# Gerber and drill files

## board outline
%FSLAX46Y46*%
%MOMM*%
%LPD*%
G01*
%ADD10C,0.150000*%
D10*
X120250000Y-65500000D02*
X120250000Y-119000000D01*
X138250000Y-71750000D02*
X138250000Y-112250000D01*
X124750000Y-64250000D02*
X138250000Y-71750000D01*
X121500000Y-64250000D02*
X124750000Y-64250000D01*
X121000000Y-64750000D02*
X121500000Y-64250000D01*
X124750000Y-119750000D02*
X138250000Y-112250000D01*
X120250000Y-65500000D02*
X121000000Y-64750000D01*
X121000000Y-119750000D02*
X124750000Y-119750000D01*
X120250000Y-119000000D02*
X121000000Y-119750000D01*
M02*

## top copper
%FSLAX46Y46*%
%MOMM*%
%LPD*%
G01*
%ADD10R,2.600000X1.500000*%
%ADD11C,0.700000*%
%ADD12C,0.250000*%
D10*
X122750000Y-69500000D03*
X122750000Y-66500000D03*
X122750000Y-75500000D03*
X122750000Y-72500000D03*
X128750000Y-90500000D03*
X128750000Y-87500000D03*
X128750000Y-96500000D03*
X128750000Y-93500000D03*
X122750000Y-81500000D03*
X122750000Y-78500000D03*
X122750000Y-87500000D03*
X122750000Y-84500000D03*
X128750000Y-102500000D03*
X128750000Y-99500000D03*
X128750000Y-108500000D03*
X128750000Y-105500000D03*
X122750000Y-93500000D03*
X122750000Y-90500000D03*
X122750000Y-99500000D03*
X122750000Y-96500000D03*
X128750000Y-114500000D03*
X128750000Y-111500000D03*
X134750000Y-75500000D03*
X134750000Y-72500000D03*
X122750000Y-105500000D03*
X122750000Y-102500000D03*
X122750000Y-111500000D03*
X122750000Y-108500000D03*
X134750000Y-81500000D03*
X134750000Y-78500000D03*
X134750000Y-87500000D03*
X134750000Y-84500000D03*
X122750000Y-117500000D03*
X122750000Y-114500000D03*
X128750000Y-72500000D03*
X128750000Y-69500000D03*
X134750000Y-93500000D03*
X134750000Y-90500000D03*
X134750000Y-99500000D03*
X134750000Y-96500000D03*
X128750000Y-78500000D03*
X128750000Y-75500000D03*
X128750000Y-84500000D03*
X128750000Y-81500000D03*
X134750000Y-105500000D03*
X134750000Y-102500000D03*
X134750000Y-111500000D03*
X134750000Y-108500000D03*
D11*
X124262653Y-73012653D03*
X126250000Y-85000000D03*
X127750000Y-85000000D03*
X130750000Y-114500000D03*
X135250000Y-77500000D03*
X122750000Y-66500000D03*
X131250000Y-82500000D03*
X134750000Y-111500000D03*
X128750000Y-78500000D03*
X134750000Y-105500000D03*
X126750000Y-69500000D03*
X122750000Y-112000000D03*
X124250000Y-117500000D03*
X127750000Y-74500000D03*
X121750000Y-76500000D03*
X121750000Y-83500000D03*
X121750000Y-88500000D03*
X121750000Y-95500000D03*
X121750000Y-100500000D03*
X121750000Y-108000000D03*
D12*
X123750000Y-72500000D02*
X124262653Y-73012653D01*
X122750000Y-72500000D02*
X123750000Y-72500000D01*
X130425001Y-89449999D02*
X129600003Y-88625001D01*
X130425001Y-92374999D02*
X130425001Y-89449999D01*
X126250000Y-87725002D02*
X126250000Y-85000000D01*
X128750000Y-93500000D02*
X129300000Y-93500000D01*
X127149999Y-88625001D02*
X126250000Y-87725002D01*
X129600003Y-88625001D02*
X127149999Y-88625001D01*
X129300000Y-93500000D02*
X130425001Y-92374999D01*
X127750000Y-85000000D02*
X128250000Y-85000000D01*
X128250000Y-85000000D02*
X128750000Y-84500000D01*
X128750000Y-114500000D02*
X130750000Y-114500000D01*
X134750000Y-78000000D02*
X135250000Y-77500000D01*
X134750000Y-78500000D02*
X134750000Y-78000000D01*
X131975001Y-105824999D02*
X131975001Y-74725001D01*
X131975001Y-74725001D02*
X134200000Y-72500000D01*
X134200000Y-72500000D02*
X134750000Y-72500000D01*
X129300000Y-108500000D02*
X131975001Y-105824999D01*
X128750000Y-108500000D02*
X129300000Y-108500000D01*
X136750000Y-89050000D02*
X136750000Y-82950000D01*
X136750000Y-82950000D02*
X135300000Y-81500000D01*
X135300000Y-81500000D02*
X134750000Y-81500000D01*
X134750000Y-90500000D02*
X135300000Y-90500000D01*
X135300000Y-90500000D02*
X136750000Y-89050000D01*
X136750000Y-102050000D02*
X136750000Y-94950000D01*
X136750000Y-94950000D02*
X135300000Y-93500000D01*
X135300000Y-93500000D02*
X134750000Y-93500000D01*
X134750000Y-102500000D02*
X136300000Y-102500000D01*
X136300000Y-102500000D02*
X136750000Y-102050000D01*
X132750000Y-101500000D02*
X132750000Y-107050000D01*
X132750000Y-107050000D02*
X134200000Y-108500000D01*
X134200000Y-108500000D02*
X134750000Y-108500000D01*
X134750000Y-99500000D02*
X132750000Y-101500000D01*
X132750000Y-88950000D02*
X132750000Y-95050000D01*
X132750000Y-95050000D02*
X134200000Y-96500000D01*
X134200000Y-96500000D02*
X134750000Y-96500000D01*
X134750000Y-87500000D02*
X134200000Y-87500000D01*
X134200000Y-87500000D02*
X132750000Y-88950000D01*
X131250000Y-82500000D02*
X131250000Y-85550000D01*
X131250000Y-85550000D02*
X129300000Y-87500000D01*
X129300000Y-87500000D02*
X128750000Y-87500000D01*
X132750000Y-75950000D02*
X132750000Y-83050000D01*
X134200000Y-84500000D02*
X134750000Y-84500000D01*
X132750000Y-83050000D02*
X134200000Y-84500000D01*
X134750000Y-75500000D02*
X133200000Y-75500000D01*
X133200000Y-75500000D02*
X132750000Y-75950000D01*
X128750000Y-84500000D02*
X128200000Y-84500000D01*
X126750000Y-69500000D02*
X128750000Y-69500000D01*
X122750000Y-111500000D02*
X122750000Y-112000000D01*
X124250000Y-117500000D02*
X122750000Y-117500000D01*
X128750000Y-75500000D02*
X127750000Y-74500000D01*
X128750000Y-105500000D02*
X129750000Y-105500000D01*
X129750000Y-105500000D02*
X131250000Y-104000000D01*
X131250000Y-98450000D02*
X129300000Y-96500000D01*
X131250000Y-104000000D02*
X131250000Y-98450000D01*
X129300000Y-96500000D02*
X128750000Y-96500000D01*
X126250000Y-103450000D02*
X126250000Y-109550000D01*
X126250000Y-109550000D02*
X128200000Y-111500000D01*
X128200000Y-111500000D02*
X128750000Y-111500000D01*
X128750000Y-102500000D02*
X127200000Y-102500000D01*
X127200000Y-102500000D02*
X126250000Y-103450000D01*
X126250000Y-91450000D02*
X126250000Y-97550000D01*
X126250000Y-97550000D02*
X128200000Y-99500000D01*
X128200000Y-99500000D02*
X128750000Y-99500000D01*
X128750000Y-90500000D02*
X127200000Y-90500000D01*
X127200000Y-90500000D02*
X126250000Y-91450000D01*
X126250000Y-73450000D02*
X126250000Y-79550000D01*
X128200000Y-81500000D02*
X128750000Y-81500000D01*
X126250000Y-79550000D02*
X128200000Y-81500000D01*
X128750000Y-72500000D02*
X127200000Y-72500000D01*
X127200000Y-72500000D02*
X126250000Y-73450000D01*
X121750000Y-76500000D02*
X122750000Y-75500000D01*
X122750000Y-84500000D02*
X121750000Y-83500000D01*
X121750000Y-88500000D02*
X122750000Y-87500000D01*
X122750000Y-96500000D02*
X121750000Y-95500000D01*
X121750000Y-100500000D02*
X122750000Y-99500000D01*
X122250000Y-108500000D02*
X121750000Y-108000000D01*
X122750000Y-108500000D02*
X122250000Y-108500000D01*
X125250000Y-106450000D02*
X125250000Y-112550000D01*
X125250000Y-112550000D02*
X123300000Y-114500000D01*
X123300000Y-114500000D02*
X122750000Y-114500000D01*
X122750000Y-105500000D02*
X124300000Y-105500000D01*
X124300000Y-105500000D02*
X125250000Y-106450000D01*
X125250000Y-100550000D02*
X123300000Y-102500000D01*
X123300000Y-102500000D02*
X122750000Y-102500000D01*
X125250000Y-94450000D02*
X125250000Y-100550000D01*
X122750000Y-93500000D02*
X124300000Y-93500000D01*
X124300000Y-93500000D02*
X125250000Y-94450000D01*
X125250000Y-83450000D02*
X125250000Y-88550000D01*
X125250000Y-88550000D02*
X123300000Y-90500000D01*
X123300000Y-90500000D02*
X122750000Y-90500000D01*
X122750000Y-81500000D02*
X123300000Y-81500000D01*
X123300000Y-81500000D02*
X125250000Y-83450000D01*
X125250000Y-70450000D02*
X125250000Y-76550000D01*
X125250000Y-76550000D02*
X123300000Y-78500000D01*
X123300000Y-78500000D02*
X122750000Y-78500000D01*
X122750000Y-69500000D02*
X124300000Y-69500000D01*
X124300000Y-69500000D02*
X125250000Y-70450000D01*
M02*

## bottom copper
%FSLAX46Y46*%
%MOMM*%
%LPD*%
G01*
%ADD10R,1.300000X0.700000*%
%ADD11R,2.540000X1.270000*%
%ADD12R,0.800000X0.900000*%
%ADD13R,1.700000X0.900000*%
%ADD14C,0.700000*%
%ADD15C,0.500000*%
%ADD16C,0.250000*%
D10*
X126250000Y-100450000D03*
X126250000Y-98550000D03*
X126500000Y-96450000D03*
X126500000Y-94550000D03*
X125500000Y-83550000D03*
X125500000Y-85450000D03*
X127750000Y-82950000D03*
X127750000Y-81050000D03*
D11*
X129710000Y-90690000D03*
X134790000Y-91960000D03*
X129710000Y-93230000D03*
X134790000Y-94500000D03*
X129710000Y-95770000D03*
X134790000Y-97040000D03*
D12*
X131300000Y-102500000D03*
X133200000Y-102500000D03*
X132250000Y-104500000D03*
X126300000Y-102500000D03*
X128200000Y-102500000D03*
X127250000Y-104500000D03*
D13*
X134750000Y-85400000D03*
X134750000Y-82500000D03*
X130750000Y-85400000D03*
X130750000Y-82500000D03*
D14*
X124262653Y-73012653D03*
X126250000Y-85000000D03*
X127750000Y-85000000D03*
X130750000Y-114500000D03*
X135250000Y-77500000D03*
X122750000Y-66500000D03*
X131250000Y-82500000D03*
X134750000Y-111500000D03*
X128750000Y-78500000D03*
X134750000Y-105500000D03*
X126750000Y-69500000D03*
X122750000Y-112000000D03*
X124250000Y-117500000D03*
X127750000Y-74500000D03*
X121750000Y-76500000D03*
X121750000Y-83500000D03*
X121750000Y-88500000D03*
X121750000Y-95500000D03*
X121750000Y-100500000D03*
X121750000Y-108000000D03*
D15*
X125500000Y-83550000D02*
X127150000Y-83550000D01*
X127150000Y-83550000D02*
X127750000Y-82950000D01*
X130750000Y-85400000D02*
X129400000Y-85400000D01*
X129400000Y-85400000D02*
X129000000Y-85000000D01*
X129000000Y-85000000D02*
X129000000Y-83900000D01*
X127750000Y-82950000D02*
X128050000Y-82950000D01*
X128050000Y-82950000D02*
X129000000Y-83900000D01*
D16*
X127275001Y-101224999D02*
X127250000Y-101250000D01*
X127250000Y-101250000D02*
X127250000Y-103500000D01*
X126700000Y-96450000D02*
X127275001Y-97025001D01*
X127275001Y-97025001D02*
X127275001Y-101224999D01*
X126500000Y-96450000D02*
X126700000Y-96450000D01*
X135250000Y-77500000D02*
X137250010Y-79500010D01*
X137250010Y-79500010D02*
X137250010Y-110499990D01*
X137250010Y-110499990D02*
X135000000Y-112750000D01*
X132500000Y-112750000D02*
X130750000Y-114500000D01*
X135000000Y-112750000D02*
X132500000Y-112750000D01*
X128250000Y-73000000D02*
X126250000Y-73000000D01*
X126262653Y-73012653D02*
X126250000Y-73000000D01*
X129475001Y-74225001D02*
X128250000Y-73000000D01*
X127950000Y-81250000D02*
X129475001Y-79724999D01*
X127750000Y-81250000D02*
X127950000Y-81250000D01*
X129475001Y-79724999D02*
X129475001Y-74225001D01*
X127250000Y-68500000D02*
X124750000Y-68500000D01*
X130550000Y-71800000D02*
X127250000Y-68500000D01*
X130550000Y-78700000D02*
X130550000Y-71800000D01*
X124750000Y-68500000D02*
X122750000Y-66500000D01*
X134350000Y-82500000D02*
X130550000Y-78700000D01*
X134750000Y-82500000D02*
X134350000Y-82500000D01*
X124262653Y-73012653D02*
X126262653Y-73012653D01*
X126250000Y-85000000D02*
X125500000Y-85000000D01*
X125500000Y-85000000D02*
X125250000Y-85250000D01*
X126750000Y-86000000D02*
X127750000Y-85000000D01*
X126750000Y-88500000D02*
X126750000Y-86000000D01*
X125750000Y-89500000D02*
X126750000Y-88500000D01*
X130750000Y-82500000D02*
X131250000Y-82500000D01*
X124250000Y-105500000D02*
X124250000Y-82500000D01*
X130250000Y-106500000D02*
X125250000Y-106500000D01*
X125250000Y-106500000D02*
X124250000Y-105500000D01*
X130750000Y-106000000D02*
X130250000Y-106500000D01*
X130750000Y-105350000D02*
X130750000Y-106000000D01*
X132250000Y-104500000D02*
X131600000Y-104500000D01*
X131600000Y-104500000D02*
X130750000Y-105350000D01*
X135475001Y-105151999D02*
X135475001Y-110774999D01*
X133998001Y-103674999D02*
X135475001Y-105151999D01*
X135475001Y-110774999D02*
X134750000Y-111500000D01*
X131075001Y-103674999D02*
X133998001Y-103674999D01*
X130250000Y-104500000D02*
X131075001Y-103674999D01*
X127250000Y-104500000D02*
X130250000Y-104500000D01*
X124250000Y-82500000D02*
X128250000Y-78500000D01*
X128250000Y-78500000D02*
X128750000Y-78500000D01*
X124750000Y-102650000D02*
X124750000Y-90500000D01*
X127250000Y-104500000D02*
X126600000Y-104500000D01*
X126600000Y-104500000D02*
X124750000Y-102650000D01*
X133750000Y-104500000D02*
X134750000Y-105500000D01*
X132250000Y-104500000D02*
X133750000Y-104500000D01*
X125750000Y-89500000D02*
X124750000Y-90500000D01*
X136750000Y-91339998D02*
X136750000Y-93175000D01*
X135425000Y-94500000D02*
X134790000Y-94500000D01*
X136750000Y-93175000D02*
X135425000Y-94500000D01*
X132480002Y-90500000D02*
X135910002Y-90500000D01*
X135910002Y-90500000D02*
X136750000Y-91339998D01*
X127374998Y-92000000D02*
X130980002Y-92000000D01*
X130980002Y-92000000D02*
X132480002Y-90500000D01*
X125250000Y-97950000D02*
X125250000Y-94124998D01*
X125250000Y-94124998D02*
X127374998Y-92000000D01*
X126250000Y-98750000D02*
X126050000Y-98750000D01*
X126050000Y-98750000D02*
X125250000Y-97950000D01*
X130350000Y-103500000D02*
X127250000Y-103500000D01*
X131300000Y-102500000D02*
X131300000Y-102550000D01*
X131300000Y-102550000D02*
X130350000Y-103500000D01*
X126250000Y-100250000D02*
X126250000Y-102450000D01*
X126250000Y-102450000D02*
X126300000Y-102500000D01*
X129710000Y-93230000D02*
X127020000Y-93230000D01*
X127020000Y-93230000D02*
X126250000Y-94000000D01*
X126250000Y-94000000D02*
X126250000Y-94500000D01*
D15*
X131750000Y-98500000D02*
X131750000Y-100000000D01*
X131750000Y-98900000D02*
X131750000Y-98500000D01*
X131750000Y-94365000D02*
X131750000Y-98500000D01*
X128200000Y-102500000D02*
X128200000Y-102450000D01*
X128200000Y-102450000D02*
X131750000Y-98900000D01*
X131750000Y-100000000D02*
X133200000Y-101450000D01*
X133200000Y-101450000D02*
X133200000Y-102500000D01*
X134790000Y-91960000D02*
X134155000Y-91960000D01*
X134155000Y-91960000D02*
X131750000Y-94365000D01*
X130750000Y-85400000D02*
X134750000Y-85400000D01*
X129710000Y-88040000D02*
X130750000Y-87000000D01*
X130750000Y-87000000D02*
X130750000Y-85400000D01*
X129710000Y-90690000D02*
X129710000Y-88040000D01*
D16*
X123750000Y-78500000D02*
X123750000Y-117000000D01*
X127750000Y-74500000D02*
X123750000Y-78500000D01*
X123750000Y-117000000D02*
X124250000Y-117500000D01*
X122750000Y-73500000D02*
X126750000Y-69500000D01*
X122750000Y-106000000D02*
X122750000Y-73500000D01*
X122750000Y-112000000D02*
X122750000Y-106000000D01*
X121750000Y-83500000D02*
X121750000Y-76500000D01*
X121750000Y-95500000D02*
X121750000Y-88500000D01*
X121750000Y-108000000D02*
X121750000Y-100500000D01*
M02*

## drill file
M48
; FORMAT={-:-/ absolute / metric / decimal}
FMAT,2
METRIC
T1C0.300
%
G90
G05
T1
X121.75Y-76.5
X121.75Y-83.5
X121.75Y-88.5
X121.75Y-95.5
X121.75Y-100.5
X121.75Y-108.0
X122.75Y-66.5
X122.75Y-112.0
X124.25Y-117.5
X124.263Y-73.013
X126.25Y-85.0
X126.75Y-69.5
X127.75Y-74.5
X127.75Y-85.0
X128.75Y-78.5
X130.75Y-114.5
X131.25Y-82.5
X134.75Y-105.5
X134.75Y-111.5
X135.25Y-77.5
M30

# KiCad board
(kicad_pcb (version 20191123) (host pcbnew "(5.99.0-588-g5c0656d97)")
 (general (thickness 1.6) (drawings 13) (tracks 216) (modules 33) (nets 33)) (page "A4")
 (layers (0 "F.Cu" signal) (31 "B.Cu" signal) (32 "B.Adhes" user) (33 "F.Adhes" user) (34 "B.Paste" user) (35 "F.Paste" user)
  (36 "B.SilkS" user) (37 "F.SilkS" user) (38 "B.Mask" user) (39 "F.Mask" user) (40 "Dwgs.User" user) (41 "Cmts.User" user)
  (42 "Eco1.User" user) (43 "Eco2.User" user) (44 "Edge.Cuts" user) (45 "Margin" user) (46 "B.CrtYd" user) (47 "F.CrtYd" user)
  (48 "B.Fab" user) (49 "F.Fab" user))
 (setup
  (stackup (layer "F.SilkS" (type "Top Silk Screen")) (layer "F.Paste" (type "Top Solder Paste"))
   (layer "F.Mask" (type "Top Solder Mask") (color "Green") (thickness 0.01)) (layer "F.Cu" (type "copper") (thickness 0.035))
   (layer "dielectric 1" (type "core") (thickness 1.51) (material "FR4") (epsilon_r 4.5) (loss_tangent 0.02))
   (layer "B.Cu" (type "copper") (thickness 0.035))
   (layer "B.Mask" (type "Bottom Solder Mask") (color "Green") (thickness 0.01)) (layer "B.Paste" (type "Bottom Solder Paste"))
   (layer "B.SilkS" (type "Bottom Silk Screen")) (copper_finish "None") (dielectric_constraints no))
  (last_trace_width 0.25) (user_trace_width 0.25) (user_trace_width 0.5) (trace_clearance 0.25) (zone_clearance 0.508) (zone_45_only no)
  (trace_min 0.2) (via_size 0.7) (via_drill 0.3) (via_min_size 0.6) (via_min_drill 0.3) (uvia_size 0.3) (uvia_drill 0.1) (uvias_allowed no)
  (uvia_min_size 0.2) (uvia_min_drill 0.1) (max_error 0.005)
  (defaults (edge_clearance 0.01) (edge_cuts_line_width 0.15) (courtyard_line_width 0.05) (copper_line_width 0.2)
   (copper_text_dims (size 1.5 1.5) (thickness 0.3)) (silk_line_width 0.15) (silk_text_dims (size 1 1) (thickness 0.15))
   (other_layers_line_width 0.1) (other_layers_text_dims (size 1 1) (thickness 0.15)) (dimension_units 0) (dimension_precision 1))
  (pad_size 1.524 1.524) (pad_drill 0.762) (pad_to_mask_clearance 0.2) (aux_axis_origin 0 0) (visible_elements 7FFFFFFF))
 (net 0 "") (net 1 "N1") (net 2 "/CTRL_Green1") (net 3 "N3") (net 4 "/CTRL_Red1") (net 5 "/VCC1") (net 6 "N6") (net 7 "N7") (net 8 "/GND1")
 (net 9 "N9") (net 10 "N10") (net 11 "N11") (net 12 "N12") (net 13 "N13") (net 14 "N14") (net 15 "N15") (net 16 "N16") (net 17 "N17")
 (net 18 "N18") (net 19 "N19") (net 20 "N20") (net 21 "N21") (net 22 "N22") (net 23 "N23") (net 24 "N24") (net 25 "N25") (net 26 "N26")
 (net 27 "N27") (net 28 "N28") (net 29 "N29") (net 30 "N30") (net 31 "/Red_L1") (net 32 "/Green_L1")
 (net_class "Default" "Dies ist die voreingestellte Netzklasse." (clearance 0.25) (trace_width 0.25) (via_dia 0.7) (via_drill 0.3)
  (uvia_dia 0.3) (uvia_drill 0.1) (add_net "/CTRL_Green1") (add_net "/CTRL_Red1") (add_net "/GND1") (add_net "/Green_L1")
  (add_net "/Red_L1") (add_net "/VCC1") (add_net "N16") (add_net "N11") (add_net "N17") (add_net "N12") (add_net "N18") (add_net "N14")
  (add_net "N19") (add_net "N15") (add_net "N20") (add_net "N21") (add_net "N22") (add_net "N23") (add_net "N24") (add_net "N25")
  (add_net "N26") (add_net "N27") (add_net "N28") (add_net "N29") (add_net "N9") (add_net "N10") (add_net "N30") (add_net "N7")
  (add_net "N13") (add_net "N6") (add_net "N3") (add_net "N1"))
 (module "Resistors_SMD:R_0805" (layer "B.Cu") (at 126.25 99.5 90)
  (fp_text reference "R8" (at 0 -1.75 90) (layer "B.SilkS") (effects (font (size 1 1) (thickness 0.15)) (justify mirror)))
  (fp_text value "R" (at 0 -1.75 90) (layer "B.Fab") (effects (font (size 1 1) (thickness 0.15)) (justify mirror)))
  (pad "1" smd rect (at -0.95 0 90) (size 0.7 1.3) (layers "B.Cu" "B.Paste" "B.Mask") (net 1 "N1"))
  (pad "2" smd rect (at 0.95 0 90) (size 0.7 1.3) (layers "B.Cu" "B.Paste" "B.Mask") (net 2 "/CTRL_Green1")))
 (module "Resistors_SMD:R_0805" (layer "B.Cu") (at 126.5 95.5 90)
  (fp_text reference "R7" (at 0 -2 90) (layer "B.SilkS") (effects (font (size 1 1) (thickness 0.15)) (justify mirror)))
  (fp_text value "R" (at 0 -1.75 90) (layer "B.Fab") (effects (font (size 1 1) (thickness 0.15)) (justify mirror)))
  (pad "1" smd rect (at -0.95 0 90) (size 0.7 1.3) (layers "B.Cu" "B.Paste" "B.Mask") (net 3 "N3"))
  (pad "2" smd rect (at 0.95 0 90) (size 0.7 1.3) (layers "B.Cu" "B.Paste" "B.Mask") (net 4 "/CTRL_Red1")))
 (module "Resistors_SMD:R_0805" (layer "B.Cu") (at 125.5 84.5 -90)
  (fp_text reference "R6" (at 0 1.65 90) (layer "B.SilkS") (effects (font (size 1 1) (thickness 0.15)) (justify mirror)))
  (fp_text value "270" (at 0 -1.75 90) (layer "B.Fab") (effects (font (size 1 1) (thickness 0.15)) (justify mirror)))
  (pad "1" smd rect (at -0.95 0 270) (size 0.7 1.3) (layers "B.Cu" "B.Paste" "B.Mask") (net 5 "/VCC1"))
  (pad "2" smd rect (at 0.95 0 270) (size 0.7 1.3) (layers "B.Cu" "B.Paste" "B.Mask") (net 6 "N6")))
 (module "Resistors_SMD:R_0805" (layer "B.Cu") (at 127.75 82 90)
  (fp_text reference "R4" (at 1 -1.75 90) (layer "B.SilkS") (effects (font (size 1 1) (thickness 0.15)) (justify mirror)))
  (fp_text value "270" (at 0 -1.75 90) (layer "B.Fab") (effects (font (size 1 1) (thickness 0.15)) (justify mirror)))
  (pad "1" smd rect (at -0.95 0 90) (size 0.7 1.3) (layers "B.Cu" "B.Paste" "B.Mask") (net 5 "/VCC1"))
  (pad "2" smd rect (at 0.95 0 90) (size 0.7 1.3) (layers "B.Cu" "B.Paste" "B.Mask") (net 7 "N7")))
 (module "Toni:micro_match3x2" (layer "B.Cu") (at 132.25 94.5 -90)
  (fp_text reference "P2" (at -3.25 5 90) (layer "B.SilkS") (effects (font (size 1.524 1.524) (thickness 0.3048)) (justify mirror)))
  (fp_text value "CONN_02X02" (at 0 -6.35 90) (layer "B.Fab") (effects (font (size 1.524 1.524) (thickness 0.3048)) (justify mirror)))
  (pad "1" smd rect (at -3.81 2.54 270) (size 1.27 2.54) (layers "B.Cu" "B.Paste" "B.Mask") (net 5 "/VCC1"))
  (pad "2" smd rect (at -2.54 -2.54 270) (size 1.27 2.54) (layers "B.Cu" "B.Paste" "B.Mask") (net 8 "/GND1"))
  (pad "3" smd rect (at -1.27 2.54 270) (size 1.27 2.54) (layers "B.Cu" "B.Paste" "B.Mask") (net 4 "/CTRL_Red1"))
  (pad "4" smd rect (at 0 -2.54 270) (size 1.27 2.54) (layers "B.Cu" "B.Paste" "B.Mask") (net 2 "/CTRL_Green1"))
  (pad "5" smd rect (at 1.27 2.54 270) (size 1.27 2.54) (layers "B.Cu" "B.Paste" "B.Mask"))
  (pad "6" smd rect (at 2.54 -2.54 270) (size 1.27 2.54) (layers "B.Cu" "B.Paste" "B.Mask")))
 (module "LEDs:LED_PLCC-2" (layer "F.Cu") (at 122.75 68 90)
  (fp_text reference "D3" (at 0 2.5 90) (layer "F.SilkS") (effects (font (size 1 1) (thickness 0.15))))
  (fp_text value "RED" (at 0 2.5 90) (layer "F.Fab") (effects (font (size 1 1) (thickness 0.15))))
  (pad "1" smd rect (at -1.5 0 90) (size 1.5 2.6) (layers "F.Cu" "F.Paste" "F.Mask") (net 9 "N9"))
  (pad "2" smd rect (at 1.5 0 90) (size 1.5 2.6) (layers "F.Cu" "F.Paste" "F.Mask") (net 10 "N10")))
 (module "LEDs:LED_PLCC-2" (layer "F.Cu") (at 122.75 74 90)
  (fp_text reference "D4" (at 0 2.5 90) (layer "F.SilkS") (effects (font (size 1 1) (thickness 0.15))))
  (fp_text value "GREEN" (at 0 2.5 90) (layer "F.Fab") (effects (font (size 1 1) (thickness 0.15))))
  (pad "1" smd rect (at -1.5 0 90) (size 1.5 2.6) (layers "F.Cu" "F.Paste" "F.Mask") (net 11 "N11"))
  (pad "2" smd rect (at 1.5 0 90) (size 1.5 2.6) (layers "F.Cu" "F.Paste" "F.Mask") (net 7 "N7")))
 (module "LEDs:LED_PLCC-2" (layer "F.Cu") (at 128.75 89 90)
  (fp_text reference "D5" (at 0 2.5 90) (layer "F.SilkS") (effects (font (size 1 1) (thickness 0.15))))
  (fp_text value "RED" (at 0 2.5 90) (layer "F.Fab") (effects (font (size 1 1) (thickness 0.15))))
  (pad "1" smd rect (at -1.5 0 90) (size 1.5 2.6) (layers "F.Cu" "F.Paste" "F.Mask") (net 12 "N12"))
  (pad "2" smd rect (at 1.5 0 90) (size 1.5 2.6) (layers "F.Cu" "F.Paste" "F.Mask") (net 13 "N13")))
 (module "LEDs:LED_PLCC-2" (layer "F.Cu") (at 128.75 95 90)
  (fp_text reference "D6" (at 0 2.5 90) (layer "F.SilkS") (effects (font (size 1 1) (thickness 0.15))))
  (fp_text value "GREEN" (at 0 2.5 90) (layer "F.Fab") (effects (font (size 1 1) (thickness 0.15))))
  (pad "1" smd rect (at -1.5 0 90) (size 1.5 2.6) (layers "F.Cu" "F.Paste" "F.Mask") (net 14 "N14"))
  (pad "2" smd rect (at 1.5 0 90) (size 1.5 2.6) (layers "F.Cu" "F.Paste" "F.Mask") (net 6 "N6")))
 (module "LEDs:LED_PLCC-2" (layer "F.Cu") (at 122.75 80 90)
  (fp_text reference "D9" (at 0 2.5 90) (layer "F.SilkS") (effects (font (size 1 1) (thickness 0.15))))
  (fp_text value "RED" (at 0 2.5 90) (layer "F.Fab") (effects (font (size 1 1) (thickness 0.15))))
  (pad "1" smd rect (at -1.5 0 90) (size 1.5 2.6) (layers "F.Cu" "F.Paste" "F.Mask") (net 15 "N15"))
  (pad "2" smd rect (at 1.5 0 90) (size 1.5 2.6) (layers "F.Cu" "F.Paste" "F.Mask") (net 9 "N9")))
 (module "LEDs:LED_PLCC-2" (layer "F.Cu") (at 122.75 86 90)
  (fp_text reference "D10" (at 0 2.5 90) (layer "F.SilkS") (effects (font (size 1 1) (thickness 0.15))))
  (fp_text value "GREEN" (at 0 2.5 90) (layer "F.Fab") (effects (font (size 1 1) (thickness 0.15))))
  (pad "1" smd rect (at -1.5 0 90) (size 1.5 2.6) (layers "F.Cu" "F.Paste" "F.Mask") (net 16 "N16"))
  (pad "2" smd rect (at 1.5 0 90) (size 1.5 2.6) (layers "F.Cu" "F.Paste" "F.Mask") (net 11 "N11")))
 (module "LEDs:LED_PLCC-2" (layer "F.Cu") (at 128.75 101 90)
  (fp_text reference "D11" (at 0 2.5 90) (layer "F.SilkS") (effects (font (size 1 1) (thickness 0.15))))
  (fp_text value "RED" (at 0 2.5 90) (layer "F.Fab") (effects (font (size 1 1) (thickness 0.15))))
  (pad "1" smd rect (at -1.5 0 90) (size 1.5 2.6) (layers "F.Cu" "F.Paste" "F.Mask") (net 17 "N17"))
  (pad "2" smd rect (at 1.5 0 90) (size 1.5 2.6) (layers "F.Cu" "F.Paste" "F.Mask") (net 12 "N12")))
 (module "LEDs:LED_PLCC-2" (layer "F.Cu") (at 128.75 107 90)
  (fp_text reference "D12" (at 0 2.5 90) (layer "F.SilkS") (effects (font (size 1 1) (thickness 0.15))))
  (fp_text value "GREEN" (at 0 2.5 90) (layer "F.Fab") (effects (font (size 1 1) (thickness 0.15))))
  (pad "1" smd rect (at -1.5 0 90) (size 1.5 2.6) (layers "F.Cu" "F.Paste" "F.Mask") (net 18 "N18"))
  (pad "2" smd rect (at 1.5 0 90) (size 1.5 2.6) (layers "F.Cu" "F.Paste" "F.Mask") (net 14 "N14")))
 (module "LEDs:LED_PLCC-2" (layer "F.Cu") (at 122.75 92 90)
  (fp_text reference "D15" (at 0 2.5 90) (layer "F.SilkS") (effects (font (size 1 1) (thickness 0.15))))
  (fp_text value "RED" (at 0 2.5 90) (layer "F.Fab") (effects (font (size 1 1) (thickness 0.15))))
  (pad "1" smd rect (at -1.5 0 90) (size 1.5 2.6) (layers "F.Cu" "F.Paste" "F.Mask") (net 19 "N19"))
  (pad "2" smd rect (at 1.5 0 90) (size 1.5 2.6) (layers "F.Cu" "F.Paste" "F.Mask") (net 15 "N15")))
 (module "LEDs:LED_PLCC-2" (layer "F.Cu") (at 122.75 98 90)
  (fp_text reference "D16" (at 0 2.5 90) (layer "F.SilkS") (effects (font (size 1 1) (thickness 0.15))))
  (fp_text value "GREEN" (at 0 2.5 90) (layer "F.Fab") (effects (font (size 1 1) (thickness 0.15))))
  (pad "1" smd rect (at -1.5 0 90) (size 1.5 2.6) (layers "F.Cu" "F.Paste" "F.Mask") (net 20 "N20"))
  (pad "2" smd rect (at 1.5 0 90) (size 1.5 2.6) (layers "F.Cu" "F.Paste" "F.Mask") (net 16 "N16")))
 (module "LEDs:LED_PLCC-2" (layer "F.Cu") (at 128.75 113 90)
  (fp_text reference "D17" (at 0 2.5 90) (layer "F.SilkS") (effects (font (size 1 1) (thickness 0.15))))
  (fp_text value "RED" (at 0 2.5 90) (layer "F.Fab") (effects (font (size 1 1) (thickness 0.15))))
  (pad "1" smd rect (at -1.5 0 90) (size 1.5 2.6) (layers "F.Cu" "F.Paste" "F.Mask") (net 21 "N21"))
  (pad "2" smd rect (at 1.5 0 90) (size 1.5 2.6) (layers "F.Cu" "F.Paste" "F.Mask") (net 17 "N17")))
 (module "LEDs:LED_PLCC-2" (layer "F.Cu") (at 134.75 74 90)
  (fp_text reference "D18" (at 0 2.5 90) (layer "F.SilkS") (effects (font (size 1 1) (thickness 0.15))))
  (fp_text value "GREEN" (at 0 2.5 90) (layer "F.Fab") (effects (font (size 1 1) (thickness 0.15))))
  (pad "1" smd rect (at -1.5 0 90) (size 1.5 2.6) (layers "F.Cu" "F.Paste" "F.Mask") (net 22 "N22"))
  (pad "2" smd rect (at 1.5 0 90) (size 1.5 2.6) (layers "F.Cu" "F.Paste" "F.Mask") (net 18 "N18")))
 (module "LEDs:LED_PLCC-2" (layer "F.Cu") (at 122.75 104 90)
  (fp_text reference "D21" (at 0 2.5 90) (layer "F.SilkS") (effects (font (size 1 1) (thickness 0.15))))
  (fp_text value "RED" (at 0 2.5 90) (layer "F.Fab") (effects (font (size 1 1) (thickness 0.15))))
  (pad "1" smd rect (at -1.5 0 90) (size 1.5 2.6) (layers "F.Cu" "F.Paste" "F.Mask") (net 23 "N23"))
  (pad "2" smd rect (at 1.5 0 90) (size 1.5 2.6) (layers "F.Cu" "F.Paste" "F.Mask") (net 19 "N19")))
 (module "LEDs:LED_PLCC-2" (layer "F.Cu") (at 122.75 110 90)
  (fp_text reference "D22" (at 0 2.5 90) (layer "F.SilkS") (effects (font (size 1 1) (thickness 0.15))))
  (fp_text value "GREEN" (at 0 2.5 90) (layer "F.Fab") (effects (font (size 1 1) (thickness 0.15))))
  (pad "1" smd rect (at -1.5 0 90) (size 1.5 2.6) (layers "F.Cu" "F.Paste" "F.Mask") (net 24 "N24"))
  (pad "2" smd rect (at 1.5 0 90) (size 1.5 2.6) (layers "F.Cu" "F.Paste" "F.Mask") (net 20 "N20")))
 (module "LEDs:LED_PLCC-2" (layer "F.Cu") (at 134.75 80 90)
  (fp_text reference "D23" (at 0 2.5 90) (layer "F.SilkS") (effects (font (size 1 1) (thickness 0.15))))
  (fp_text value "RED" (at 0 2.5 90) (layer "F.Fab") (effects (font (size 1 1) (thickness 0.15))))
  (pad "1" smd rect (at -1.5 0 90) (size 1.5 2.6) (layers "F.Cu" "F.Paste" "F.Mask") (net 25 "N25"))
  (pad "2" smd rect (at 1.5 0 90) (size 1.5 2.6) (layers "F.Cu" "F.Paste" "F.Mask") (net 21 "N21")))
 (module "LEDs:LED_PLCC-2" (layer "F.Cu") (at 134.75 86 90)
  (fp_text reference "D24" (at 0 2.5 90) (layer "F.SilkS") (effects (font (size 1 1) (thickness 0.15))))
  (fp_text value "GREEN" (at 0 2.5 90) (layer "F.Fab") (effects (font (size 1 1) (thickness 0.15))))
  (pad "1" smd rect (at -1.5 0 90) (size 1.5 2.6) (layers "F.Cu" "F.Paste" "F.Mask") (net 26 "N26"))
  (pad "2" smd rect (at 1.5 0 90) (size 1.5 2.6) (layers "F.Cu" "F.Paste" "F.Mask") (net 22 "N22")))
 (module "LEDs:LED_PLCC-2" (layer "F.Cu") (at 122.75 116 90)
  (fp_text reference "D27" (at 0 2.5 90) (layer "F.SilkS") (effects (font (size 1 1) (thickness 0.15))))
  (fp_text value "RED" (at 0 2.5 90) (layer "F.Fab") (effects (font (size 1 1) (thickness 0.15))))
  (pad "1" smd rect (at -1.5 0 90) (size 1.5 2.6) (layers "F.Cu" "F.Paste" "F.Mask") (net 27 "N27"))
  (pad "2" smd rect (at 1.5 0 90) (size 1.5 2.6) (layers "F.Cu" "F.Paste" "F.Mask") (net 23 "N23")))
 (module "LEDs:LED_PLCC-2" (layer "F.Cu") (at 128.75 71 90)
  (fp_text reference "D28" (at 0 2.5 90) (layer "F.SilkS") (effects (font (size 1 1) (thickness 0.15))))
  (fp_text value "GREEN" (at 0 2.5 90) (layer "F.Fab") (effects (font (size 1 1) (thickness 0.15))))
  (pad "1" smd rect (at -1.5 0 90) (size 1.5 2.6) (layers "F.Cu" "F.Paste" "F.Mask") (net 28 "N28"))
  (pad "2" smd rect (at 1.5 0 90) (size 1.5 2.6) (layers "F.Cu" "F.Paste" "F.Mask") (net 24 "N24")))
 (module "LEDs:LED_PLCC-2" (layer "F.Cu") (at 134.75 92 90)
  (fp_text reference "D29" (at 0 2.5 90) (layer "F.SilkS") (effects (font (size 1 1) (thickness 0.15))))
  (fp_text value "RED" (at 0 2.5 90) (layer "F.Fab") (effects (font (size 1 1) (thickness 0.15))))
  (pad "1" smd rect (at -1.5 0 90) (size 1.5 2.6) (layers "F.Cu" "F.Paste" "F.Mask") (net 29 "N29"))
  (pad "2" smd rect (at 1.5 0 90) (size 1.5 2.6) (layers "F.Cu" "F.Paste" "F.Mask") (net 25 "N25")))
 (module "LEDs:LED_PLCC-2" (layer "F.Cu") (at 134.75 98 90)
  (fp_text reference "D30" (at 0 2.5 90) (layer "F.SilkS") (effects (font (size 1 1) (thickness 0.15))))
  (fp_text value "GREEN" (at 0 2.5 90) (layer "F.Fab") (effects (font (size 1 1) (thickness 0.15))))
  (pad "1" smd rect (at -1.5 0 90) (size 1.5 2.6) (layers "F.Cu" "F.Paste" "F.Mask") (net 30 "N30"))
  (pad "2" smd rect (at 1.5 0 90) (size 1.5 2.6) (layers "F.Cu" "F.Paste" "F.Mask") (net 26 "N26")))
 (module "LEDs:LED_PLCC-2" (layer "F.Cu") (at 128.75 77 90)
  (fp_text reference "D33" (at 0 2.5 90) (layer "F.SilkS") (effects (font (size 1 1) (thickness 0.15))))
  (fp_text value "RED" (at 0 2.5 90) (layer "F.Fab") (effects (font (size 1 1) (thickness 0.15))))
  (pad "1" smd rect (at -1.5 0 90) (size 1.5 2.6) (layers "F.Cu" "F.Paste" "F.Mask") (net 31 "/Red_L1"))
  (pad "2" smd rect (at 1.5 0 90) (size 1.5 2.6) (layers "F.Cu" "F.Paste" "F.Mask") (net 27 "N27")))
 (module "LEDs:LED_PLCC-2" (layer "F.Cu") (at 128.75 83 90)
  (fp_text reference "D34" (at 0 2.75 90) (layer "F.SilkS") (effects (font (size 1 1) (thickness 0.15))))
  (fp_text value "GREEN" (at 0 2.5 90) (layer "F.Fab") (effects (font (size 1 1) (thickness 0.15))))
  (pad "1" smd rect (at -1.5 0 90) (size 1.5 2.6) (layers "F.Cu" "F.Paste" "F.Mask") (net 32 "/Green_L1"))
  (pad "2" smd rect (at 1.5 0 90) (size 1.5 2.6) (layers "F.Cu" "F.Paste" "F.Mask") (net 28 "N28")))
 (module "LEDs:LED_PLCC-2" (layer "F.Cu") (at 134.75 104 90)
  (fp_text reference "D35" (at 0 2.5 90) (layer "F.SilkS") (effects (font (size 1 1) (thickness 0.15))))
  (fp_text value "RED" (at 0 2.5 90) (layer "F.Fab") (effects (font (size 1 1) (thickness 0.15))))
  (pad "1" smd rect (at -1.5 0 90) (size 1.5 2.6) (layers "F.Cu" "F.Paste" "F.Mask") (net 31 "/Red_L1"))
  (pad "2" smd rect (at 1.5 0 90) (size 1.5 2.6) (layers "F.Cu" "F.Paste" "F.Mask") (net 29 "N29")))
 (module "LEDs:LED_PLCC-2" (layer "F.Cu") (at 134.75 110 90)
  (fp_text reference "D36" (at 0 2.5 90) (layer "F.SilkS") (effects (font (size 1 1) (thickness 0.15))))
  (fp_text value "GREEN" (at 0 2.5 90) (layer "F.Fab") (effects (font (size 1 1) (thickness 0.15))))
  (pad "1" smd rect (at -1.5 0 90) (size 1.5 2.6) (layers "F.Cu" "F.Paste" "F.Mask") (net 32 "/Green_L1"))
  (pad "2" smd rect (at 1.5 0 90) (size 1.5 2.6) (layers "F.Cu" "F.Paste" "F.Mask") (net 30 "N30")))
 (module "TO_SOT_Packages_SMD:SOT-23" (layer "B.Cu") (at 132.25 103.5 -90)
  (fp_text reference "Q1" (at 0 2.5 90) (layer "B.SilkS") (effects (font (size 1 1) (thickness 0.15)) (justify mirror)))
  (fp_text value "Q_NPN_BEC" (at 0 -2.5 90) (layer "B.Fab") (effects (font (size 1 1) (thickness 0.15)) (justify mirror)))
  (pad "1" smd rect (at -1 0.95 270) (size 0.9 0.8) (layers "B.Cu" "B.Paste" "B.Mask") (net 3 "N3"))
  (pad "2" smd rect (at -1 -0.95 270) (size 0.9 0.8) (layers "B.Cu" "B.Paste" "B.Mask") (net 8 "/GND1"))
  (pad "3" smd rect (at 1 0 270) (size 0.9 0.8) (layers "B.Cu" "B.Paste" "B.Mask") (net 31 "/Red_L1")))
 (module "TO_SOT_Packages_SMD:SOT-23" (layer "B.Cu") (at 127.25 103.5 -90)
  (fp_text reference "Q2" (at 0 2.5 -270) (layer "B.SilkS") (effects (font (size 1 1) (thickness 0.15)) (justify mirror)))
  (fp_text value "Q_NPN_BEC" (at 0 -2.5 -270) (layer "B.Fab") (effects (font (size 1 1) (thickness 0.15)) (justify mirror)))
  (pad "1" smd rect (at -1 0.95 270) (size 0.9 0.8) (layers "B.Cu" "B.Paste" "B.Mask") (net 1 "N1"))
  (pad "2" smd rect (at -1 -0.95 270) (size 0.9 0.8) (layers "B.Cu" "B.Paste" "B.Mask") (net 8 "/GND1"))
  (pad "3" smd rect (at 1 0 270) (size 0.9 0.8) (layers "B.Cu" "B.Paste" "B.Mask") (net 32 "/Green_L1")))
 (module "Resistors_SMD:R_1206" (layer "B.Cu") (at 134.75 83.95 90)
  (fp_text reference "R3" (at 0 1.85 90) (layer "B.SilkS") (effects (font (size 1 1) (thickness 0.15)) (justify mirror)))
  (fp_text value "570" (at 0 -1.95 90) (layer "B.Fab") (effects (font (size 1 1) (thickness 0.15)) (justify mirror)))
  (pad "1" smd rect (at -1.45 0 90) (size 0.9 1.7) (layers "B.Cu" "B.Paste" "B.Mask") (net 5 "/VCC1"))
  (pad "2" smd rect (at 1.45 0 90) (size 0.9 1.7) (layers "B.Cu" "B.Paste" "B.Mask") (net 10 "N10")))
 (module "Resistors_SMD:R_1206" (layer "B.Cu") (at 130.75 83.95 90)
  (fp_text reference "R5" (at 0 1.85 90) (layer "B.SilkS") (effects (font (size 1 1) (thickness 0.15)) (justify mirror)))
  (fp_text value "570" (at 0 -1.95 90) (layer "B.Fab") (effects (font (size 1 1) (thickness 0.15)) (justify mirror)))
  (pad "1" smd rect (at -1.45 0 90) (size 0.9 1.7) (layers "B.Cu" "B.Paste" "B.Mask") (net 5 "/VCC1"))
  (pad "2" smd rect (at 1.45 0 90) (size 0.9 1.7) (layers "B.Cu" "B.Paste" "B.Mask") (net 13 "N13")))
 (gr_line (start 120.25 65.5) (end 120.25 119) (layer "Edge.Cuts") (width 0.15))
 (gr_line (start 138.25 71.75) (end 138.25 112.25) (layer "Edge.Cuts") (width 0.15))
 (gr_line (start 124.75 64.25) (end 138.25 71.75) (layer "Edge.Cuts") (width 0.15))
 (gr_line (start 121.5 64.25) (end 124.75 64.25) (layer "Edge.Cuts") (width 0.15))
 (gr_line (start 121 64.75) (end 121.5 64.25) (layer "Edge.Cuts") (width 0.15))
 (gr_line (start 124.75 119.75) (end 138.25 112.25) (layer "Edge.Cuts") (width 0.15))
 (gr_line (start 120.25 65.5) (end 121 64.75) (layer "Edge.Cuts") (width 0.15))
 (gr_line (start 121 119.75) (end 124.75 119.75) (layer "Edge.Cuts") (width 0.15))
 (gr_line (start 120.25 119) (end 121 119.75) (layer "Edge.Cuts") (width 0.15))
 (segment (start 125.5 83.55) (end 127.15 83.55) (width 0.5) (layer "B.Cu") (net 5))
 (segment (start 127.15 83.55) (end 127.75 82.95) (width 0.5) (layer "B.Cu") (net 5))
 (segment (start 130.75 85.4) (end 129.4 85.4) (width 0.5) (layer "B.Cu") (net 5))
 (segment (start 129.4 85.4) (end 129 85) (width 0.5) (layer "B.Cu") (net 5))
 (segment (start 129 85) (end 129 83.9) (width 0.5) (layer "B.Cu") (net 5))
 (segment (start 127.75 82.95) (end 128.05 82.95) (width 0.5) (layer "B.Cu") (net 5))
 (segment (start 128.05 82.95) (end 129 83.9) (width 0.5) (layer "B.Cu") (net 5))
 (segment (start 127.275001 101.224999) (end 127.25 101.25) (width 0.25) (layer "B.Cu") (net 3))
 (segment (start 127.25 101.25) (end 127.25 103.5) (width 0.25) (layer "B.Cu") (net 3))
 (segment (start 126.7 96.45) (end 127.275001 97.025001) (width 0.25) (layer "B.Cu") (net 3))
 (segment (start 127.275001 97.025001) (end 127.275001 101.224999) (width 0.25) (layer "B.Cu") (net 3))
 (segment (start 126.5 96.45) (end 126.7 96.45) (width 0.25) (layer "B.Cu") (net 3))
 (segment (start 135.25 77.5) (end 137.25001 79.50001) (width 0.25) (layer "B.Cu") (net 21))
 (segment (start 137.25001 79.50001) (end 137.25001 110.49999) (width 0.25) (layer "B.Cu") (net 21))
 (segment (start 137.25001 110.49999) (end 135 112.75) (width 0.25) (layer "B.Cu") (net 21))
 (segment (start 132.5 112.75) (end 130.75 114.5) (width 0.25) (layer "B.Cu") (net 21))
 (segment (start 135 112.75) (end 132.5 112.75) (width 0.25) (layer "B.Cu") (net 21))
 (segment (start 128.25 73) (end 126.25 73) (width 0.25) (layer "B.Cu") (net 7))
 (segment (start 126.262653 73.012653) (end 126.25 73) (width 0.25) (layer "B.Cu") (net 7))
 (segment (start 129.475001 74.225001) (end 128.25 73) (width 0.25) (layer "B.Cu") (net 7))
 (segment (start 127.95 81.25) (end 129.475001 79.724999) (width 0.25) (layer "B.Cu") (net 7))
 (segment (start 127.75 81.25) (end 127.95 81.25) (width 0.25) (layer "B.Cu") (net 7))
 (segment (start 129.475001 79.724999) (end 129.475001 74.225001) (width 0.25) (layer "B.Cu") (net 7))
 (segment (start 127.25 68.5) (end 124.75 68.5) (width 0.25) (layer "B.Cu") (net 10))
 (segment (start 130.55 71.8) (end 127.25 68.5) (width 0.25) (layer "B.Cu") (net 10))
 (segment (start 130.55 78.7) (end 130.55 71.8) (width 0.25) (layer "B.Cu") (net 10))
 (segment (start 124.75 68.5) (end 122.75 66.5) (width 0.25) (layer "B.Cu") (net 10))
 (segment (start 134.35 82.5) (end 130.55 78.7) (width 0.25) (layer "B.Cu") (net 10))
 (segment (start 134.75 82.5) (end 134.35 82.5) (width 0.25) (layer "B.Cu") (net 10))
 (segment (start 124.262653 73.012653) (end 126.262653 73.012653) (width 0.25) (layer "B.Cu") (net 7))
 (segment (start 123.75 72.5) (end 124.262653 73.012653) (width 0.25) (layer "F.Cu") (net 7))
 (segment (start 122.75 72.5) (end 123.75 72.5) (width 0.25) (layer "F.Cu") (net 7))
 (via (at 124.262653 73.012653) (size 0.7) (drill 0.3) (layers "F.Cu" "B.Cu") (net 7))
 (segment (start 126.25 85) (end 125.5 85) (width 0.25) (layer "B.Cu") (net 6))
 (segment (start 125.5 85) (end 125.25 85.25) (width 0.25) (layer "B.Cu") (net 6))
 (segment (start 130.425001 89.449999) (end 129.600003 88.625001) (width 0.25) (layer "F.Cu") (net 6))
 (segment (start 130.425001 92.374999) (end 130.425001 89.449999) (width 0.25) (layer "F.Cu") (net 6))
 (segment (start 126.25 87.725002) (end 126.25 85) (width 0.25) (layer "F.Cu") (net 6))
 (via (at 126.25 85) (size 0.7) (drill 0.3) (layers "F.Cu" "B.Cu") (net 6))
 (segment (start 128.75 93.5) (end 129.3 93.5) (width 0.25) (layer "F.Cu") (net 6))
 (segment (start 127.149999 88.625001) (end 126.25 87.725002) (width 0.25) (layer "F.Cu") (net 6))
 (segment (start 129.600003 88.625001) (end 127.149999 88.625001) (width 0.25) (layer "F.Cu") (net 6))
 (segment (start 129.3 93.5) (end 130.425001 92.374999) (width 0.25) (layer "F.Cu") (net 6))
 (segment (start 127.75 85) (end 128.25 85) (width 0.25) (layer "F.Cu") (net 32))
 (segment (start 128.25 85) (end 128.75 84.5) (width 0.25) (layer "F.Cu") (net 32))
 (segment (start 126.75 86) (end 127.75 85) (width 0.25) (layer "B.Cu") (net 32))
 (via (at 127.75 85) (size 0.7) (drill 0.3) (layers "F.Cu" "B.Cu") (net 32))
 (segment (start 126.75 88.5) (end 126.75 86) (width 0.25) (layer "B.Cu") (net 32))
 (segment (start 125.75 89.5) (end 126.75 88.5) (width 0.25) (layer "B.Cu") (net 32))
 (segment (start 128.75 114.5) (end 130.75 114.5) (width 0.25) (layer "F.Cu") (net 21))
 (via (at 130.75 114.5) (size 0.7) (drill 0.3) (layers "F.Cu" "B.Cu") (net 21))
 (segment (start 134.75 78) (end 135.25 77.5) (width 0.25) (layer "F.Cu") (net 21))
 (via (at 135.25 77.5) (size 0.7) (drill 0.3) (layers "F.Cu" "B.Cu") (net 21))
 (segment (start 134.75 78.5) (end 134.75 78) (width 0.25) (layer "F.Cu") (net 21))
 (segment (start 131.975001 105.824999) (end 131.975001 74.725001) (width 0.25) (layer "F.Cu") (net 18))
 (segment (start 131.975001 74.725001) (end 134.2 72.5) (width 0.25) (layer "F.Cu") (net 18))
 (segment (start 134.2 72.5) (end 134.75 72.5) (width 0.25) (layer "F.Cu") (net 18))
 (segment (start 129.3 108.5) (end 131.975001 105.824999) (width 0.25) (layer "F.Cu") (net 18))
 (segment (start 128.75 108.5) (end 129.3 108.5) (width 0.25) (layer "F.Cu") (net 18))
 (segment (start 136.75 89.05) (end 136.75 82.95) (width 0.25) (layer "F.Cu") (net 25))
 (segment (start 136.75 82.95) (end 135.3 81.5) (width 0.25) (layer "F.Cu") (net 25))
 (segment (start 135.3 81.5) (end 134.75 81.5) (width 0.25) (layer "F.Cu") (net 25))
 (segment (start 134.75 90.5) (end 135.3 90.5) (width 0.25) (layer "F.Cu") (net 25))
 (segment (start 135.3 90.5) (end 136.75 89.05) (width 0.25) (layer "F.Cu") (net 25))
 (segment (start 136.75 102.05) (end 136.75 94.95) (width 0.25) (layer "F.Cu") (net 29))
 (segment (start 136.75 94.95) (end 135.3 93.5) (width 0.25) (layer "F.Cu") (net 29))
 (segment (start 135.3 93.5) (end 134.75 93.5) (width 0.25) (layer "F.Cu") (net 29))
 (segment (start 134.75 102.5) (end 136.3 102.5) (width 0.25) (layer "F.Cu") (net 29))
 (segment (start 136.3 102.5) (end 136.75 102.05) (width 0.25) (layer "F.Cu") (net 29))
 (segment (start 132.75 101.5) (end 132.75 107.05) (width 0.25) (layer "F.Cu") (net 30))
 (segment (start 132.75 107.05) (end 134.2 108.5) (width 0.25) (layer "F.Cu") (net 30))
 (segment (start 134.2 108.5) (end 134.75 108.5) (width 0.25) (layer "F.Cu") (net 30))
 (segment (start 134.75 99.5) (end 132.75 101.5) (width 0.25) (layer "F.Cu") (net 30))
 (segment (start 132.75 88.95) (end 132.75 95.05) (width 0.25) (layer "F.Cu") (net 26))
 (segment (start 132.75 95.05) (end 134.2 96.5) (width 0.25) (layer "F.Cu") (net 26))
 (segment (start 134.2 96.5) (end 134.75 96.5) (width 0.25) (layer "F.Cu") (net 26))
 (segment (start 134.75 87.5) (end 134.2 87.5) (width 0.25) (layer "F.Cu") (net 26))
 (segment (start 134.2 87.5) (end 132.75 88.95) (width 0.25) (layer "F.Cu") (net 26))
 (via (at 122.75 66.5) (size 0.7) (drill 0.3) (layers "F.Cu" "B.Cu") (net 10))
 (segment (start 131.25 82.5) (end 131.25 85.55) (width 0.25) (layer "F.Cu") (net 13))
 (segment (start 131.25 85.55) (end 129.3 87.5) (width 0.25) (layer "F.Cu") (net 13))
 (segment (start 129.3 87.5) (end 128.75 87.5) (width 0.25) (layer "F.Cu") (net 13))
 (segment (start 130.75 82.5) (end 131.25 82.5) (width 0.25) (layer "B.Cu") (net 13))
 (via (at 131.25 82.5) (size 0.7) (drill 0.3) (layers "F.Cu" "B.Cu") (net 13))
 (segment (start 132.75 75.95) (end 132.75 83.05) (width 0.25) (layer "F.Cu") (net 22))
 (segment (start 134.2 84.5) (end 134.75 84.5) (width 0.25) (layer "F.Cu") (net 22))
 (segment (start 132.75 83.05) (end 134.2 84.5) (width 0.25) (layer "F.Cu") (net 22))
 (segment (start 134.75 75.5) (end 133.2 75.5) (width 0.25) (layer "F.Cu") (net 22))
 (segment (start 133.2 75.5) (end 132.75 75.95) (width 0.25) (layer "F.Cu") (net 22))
 (segment (start 124.25 105.5) (end 124.25 82.5) (width 0.25) (layer "B.Cu") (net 31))
 (segment (start 130.25 106.5) (end 125.25 106.5) (width 0.25) (layer "B.Cu") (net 31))
 (segment (start 125.25 106.5) (end 124.25 105.5) (width 0.25) (layer "B.Cu") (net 31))
 (segment (start 130.75 106) (end 130.25 106.5) (width 0.25) (layer "B.Cu") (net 31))
 (segment (start 130.75 105.35) (end 130.75 106) (width 0.25) (layer "B.Cu") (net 31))
 (segment (start 132.25 104.5) (end 131.6 104.5) (width 0.25) (layer "B.Cu") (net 31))
 (segment (start 131.6 104.5) (end 130.75 105.35) (width 0.25) (layer "B.Cu") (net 31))
 (segment (start 135.475001 105.151999) (end 135.475001 110.774999) (width 0.25) (layer "B.Cu") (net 32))
 (segment (start 133.998001 103.674999) (end 135.475001 105.151999) (width 0.25) (layer "B.Cu") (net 32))
 (segment (start 135.475001 110.774999) (end 134.75 111.5) (width 0.25) (layer "B.Cu") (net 32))
 (segment (start 131.075001 103.674999) (end 133.998001 103.674999) (width 0.25) (layer "B.Cu") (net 32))
 (segment (start 130.25 104.5) (end 131.075001 103.674999) (width 0.25) (layer "B.Cu") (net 32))
 (via (at 134.75 111.5) (size 0.7) (drill 0.3) (layers "F.Cu" "B.Cu") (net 32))
 (segment (start 127.25 104.5) (end 130.25 104.5) (width 0.25) (layer "B.Cu") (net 32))
 (segment (start 124.25 82.5) (end 128.25 78.5) (width 0.25) (layer "B.Cu") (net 31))
 (segment (start 128.25 78.5) (end 128.75 78.5) (width 0.25) (layer "B.Cu") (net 31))
 (segment (start 124.75 102.65) (end 124.75 90.5) (width 0.25) (layer "B.Cu") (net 32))
 (segment (start 127.25 104.5) (end 126.6 104.5) (width 0.25) (layer "B.Cu") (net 32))
 (segment (start 126.6 104.5) (end 124.75 102.65) (width 0.25) (layer "B.Cu") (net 32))
 (via (at 128.75 78.5) (size 0.7) (drill 0.3) (layers "F.Cu" "B.Cu") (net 31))
 (segment (start 133.75 104.5) (end 134.75 105.5) (width 0.25) (layer "B.Cu") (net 31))
 (segment (start 132.25 104.5) (end 133.75 104.5) (width 0.25) (layer "B.Cu") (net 31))
 (via (at 134.75 105.5) (size 0.7) (drill 0.3) (layers "F.Cu" "B.Cu") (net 31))
 (segment (start 125.75 89.5) (end 124.75 90.5) (width 0.25) (layer "B.Cu") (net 32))
 (segment (start 128.75 84.5) (end 128.2 84.5) (width 0.25) (layer "F.Cu") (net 32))
 (segment (start 136.75 91.339998) (end 136.75 93.175) (width 0.25) (layer "B.Cu") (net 2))
 (segment (start 135.425 94.5) (end 134.79 94.5) (width 0.25) (layer "B.Cu") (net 2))
 (segment (start 136.75 93.175) (end 135.425 94.5) (width 0.25) (layer "B.Cu") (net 2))
 (segment (start 132.480002 90.5) (end 135.910002 90.5) (width 0.25) (layer "B.Cu") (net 2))
 (segment (start 135.910002 90.5) (end 136.75 91.339998) (width 0.25) (layer "B.Cu") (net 2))
 (segment (start 127.374998 92) (end 130.980002 92) (width 0.25) (layer "B.Cu") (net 2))
 (segment (start 130.980002 92) (end 132.480002 90.5) (width 0.25) (layer "B.Cu") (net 2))
 (segment (start 125.25 97.95) (end 125.25 94.124998) (width 0.25) (layer "B.Cu") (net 2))
 (segment (start 125.25 94.124998) (end 127.374998 92) (width 0.25) (layer "B.Cu") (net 2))
 (segment (start 126.25 98.75) (end 126.05 98.75) (width 0.25) (layer "B.Cu") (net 2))
 (segment (start 126.05 98.75) (end 125.25 97.95) (width 0.25) (layer "B.Cu") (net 2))
 (segment (start 130.35 103.5) (end 127.25 103.5) (width 0.25) (layer "B.Cu") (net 3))
 (segment (start 131.3 102.5) (end 131.3 102.55) (width 0.25) (layer "B.Cu") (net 3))
 (segment (start 131.3 102.55) (end 130.35 103.5) (width 0.25) (layer "B.Cu") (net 3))
 (segment (start 126.25 100.25) (end 126.25 102.45) (width 0.25) (layer "B.Cu") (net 1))
 (segment (start 126.25 102.45) (end 126.3 102.5) (width 0.25) (layer "B.Cu") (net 1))
 (segment (start 129.71 93.23) (end 127.02 93.23) (width 0.25) (layer "B.Cu") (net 4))
 (segment (start 127.02 93.23) (end 126.25 94) (width 0.25) (layer "B.Cu") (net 4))
 (segment (start 126.25 94) (end 126.25 94.5) (width 0.25) (layer "B.Cu") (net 4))
 (segment (start 131.75 98.5) (end 131.75 100) (width 0.5) (layer "B.Cu") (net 8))
 (segment (start 131.75 98.9) (end 131.75 98.5) (width 0.5) (layer "B.Cu") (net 8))
 (segment (start 131.75 94.365) (end 131.75 98.5) (width 0.5) (layer "B.Cu") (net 8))
 (segment (start 128.2 102.5) (end 128.2 102.45) (width 0.5) (layer "B.Cu") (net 8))
 (segment (start 128.2 102.45) (end 131.75 98.9) (width 0.5) (layer "B.Cu") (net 8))
 (segment (start 131.75 100) (end 133.2 101.45) (width 0.5) (layer "B.Cu") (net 8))
 (segment (start 133.2 101.45) (end 133.2 102.5) (width 0.5) (layer "B.Cu") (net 8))
 (segment (start 134.79 91.96) (end 134.155 91.96) (width 0.5) (layer "B.Cu") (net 8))
 (segment (start 134.155 91.96) (end 131.75 94.365) (width 0.5) (layer "B.Cu") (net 8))
 (segment (start 130.75 85.4) (end 134.75 85.4) (width 0.5) (layer "B.Cu") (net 5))
 (segment (start 129.71 88.04) (end 130.75 87) (width 0.5) (layer "B.Cu") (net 5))
 (segment (start 130.75 87) (end 130.75 85.4) (width 0.5) (layer "B.Cu") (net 5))
 (segment (start 129.71 90.69) (end 129.71 88.04) (width 0.5) (layer "B.Cu") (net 5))
 (segment (start 123.75 78.5) (end 123.75 117) (width 0.25) (layer "B.Cu") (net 27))
 (segment (start 127.75 74.5) (end 123.75 78.5) (width 0.25) (layer "B.Cu") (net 27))
 (segment (start 123.75 117) (end 124.25 117.5) (width 0.25) (layer "B.Cu") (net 27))
 (segment (start 126.75 69.5) (end 128.75 69.5) (width 0.25) (layer "F.Cu") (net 24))
 (segment (start 122.75 73.5) (end 126.75 69.5) (width 0.25) (layer "B.Cu") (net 24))
 (segment (start 122.75 106) (end 122.75 73.5) (width 0.25) (layer "B.Cu") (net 24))
 (via (at 126.75 69.5) (size 0.7) (drill 0.3) (layers "F.Cu" "B.Cu") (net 24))
 (segment (start 122.75 112) (end 122.75 106) (width 0.25) (layer "B.Cu") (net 24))
 (segment (start 122.75 111.5) (end 122.75 112) (width 0.25) (layer "F.Cu") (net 24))
 (via (at 122.75 112) (size 0.7) (drill 0.3) (layers "F.Cu" "B.Cu") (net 24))
 (segment (start 124.25 117.5) (end 122.75 117.5) (width 0.25) (layer "F.Cu") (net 27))
 (via (at 124.25 117.5) (size 0.7) (drill 0.3) (layers "F.Cu" "B.Cu") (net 27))
 (segment (start 128.75 75.5) (end 127.75 74.5) (width 0.25) (layer "F.Cu") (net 27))
 (via (at 127.75 74.5) (size 0.7) (drill 0.3) (layers "F.Cu" "B.Cu") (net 27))
 (segment (start 128.75 105.5) (end 129.75 105.5) (width 0.25) (layer "F.Cu") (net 14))
 (segment (start 129.75 105.5) (end 131.25 104) (width 0.25) (layer "F.Cu") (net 14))
 (segment (start 131.25 98.45) (end 129.3 96.5) (width 0.25) (layer "F.Cu") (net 14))
 (segment (start 131.25 104) (end 131.25 98.45) (width 0.25) (layer "F.Cu") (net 14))
 (segment (start 129.3 96.5) (end 128.75 96.5) (width 0.25) (layer "F.Cu") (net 14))
 (segment (start 126.25 103.45) (end 126.25 109.55) (width 0.25) (layer "F.Cu") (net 17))
 (segment (start 126.25 109.55) (end 128.2 111.5) (width 0.25) (layer "F.Cu") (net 17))
 (segment (start 128.2 111.5) (end 128.75 111.5) (width 0.25) (layer "F.Cu") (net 17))
 (segment (start 128.75 102.5) (end 127.2 102.5) (width 0.25) (layer "F.Cu") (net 17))
 (segment (start 127.2 102.5) (end 126.25 103.45) (width 0.25) (layer "F.Cu") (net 17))
 (segment (start 126.25 91.45) (end 126.25 97.55) (width 0.25) (layer "F.Cu") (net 12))
 (segment (start 126.25 97.55) (end 128.2 99.5) (width 0.25) (layer "F.Cu") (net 12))
 (segment (start 128.2 99.5) (end 128.75 99.5) (width 0.25) (layer "F.Cu") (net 12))
 (segment (start 128.75 90.5) (end 127.2 90.5) (width 0.25) (layer "F.Cu") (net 12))
 (segment (start 127.2 90.5) (end 126.25 91.45) (width 0.25) (layer "F.Cu") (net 12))
 (segment (start 126.25 73.45) (end 126.25 79.55) (width 0.25) (layer "F.Cu") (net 28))
 (segment (start 128.2 81.5) (end 128.75 81.5) (width 0.25) (layer "F.Cu") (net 28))
 (segment (start 126.25 79.55) (end 128.2 81.5) (width 0.25) (layer "F.Cu") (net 28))
 (segment (start 128.75 72.5) (end 127.2 72.5) (width 0.25) (layer "F.Cu") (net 28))
 (segment (start 127.2 72.5) (end 126.25 73.45) (width 0.25) (layer "F.Cu") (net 28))
 (segment (start 121.75 76.5) (end 122.75 75.5) (width 0.25) (layer "F.Cu") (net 11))
 (segment (start 121.75 83.5) (end 121.75 76.5) (width 0.25) (layer "B.Cu") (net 11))
 (via (at 121.75 76.5) (size 0.7) (drill 0.3) (layers "F.Cu" "B.Cu") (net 11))
 (segment (start 122.75 84.5) (end 121.75 83.5) (width 0.25) (layer "F.Cu") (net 11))
 (via (at 121.75 83.5) (size 0.7) (drill 0.3) (layers "F.Cu" "B.Cu") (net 11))
 (segment (start 121.75 88.5) (end 122.75 87.5) (width 0.25) (layer "F.Cu") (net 16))
 (segment (start 121.75 95.5) (end 121.75 88.5) (width 0.25) (layer "B.Cu") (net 16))
 (via (at 121.75 88.5) (size 0.7) (drill 0.3) (layers "F.Cu" "B.Cu") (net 16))
 (segment (start 122.75 96.5) (end 121.75 95.5) (width 0.25) (layer "F.Cu") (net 16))
 (via (at 121.75 95.5) (size 0.7) (drill 0.3) (layers "F.Cu" "B.Cu") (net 16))
 (segment (start 121.75 100.5) (end 122.75 99.5) (width 0.25) (layer "F.Cu") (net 20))
 (segment (start 121.75 108) (end 121.75 100.5) (width 0.25) (layer "B.Cu") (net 20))
 (via (at 121.75 100.5) (size 0.7) (drill 0.3) (layers "F.Cu" "B.Cu") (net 20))
 (segment (start 122.25 108.5) (end 121.75 108) (width 0.25) (layer "F.Cu") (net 20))
 (segment (start 122.75 108.5) (end 122.25 108.5) (width 0.25) (layer "F.Cu") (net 20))
 (via (at 121.75 108) (size 0.7) (drill 0.3) (layers "F.Cu" "B.Cu") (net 20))
 (segment (start 125.25 106.45) (end 125.25 112.55) (width 0.25) (layer "F.Cu") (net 23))
 (segment (start 125.25 112.55) (end 123.3 114.5) (width 0.25) (layer "F.Cu") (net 23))
 (segment (start 123.3 114.5) (end 122.75 114.5) (width 0.25) (layer "F.Cu") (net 23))
 (segment (start 122.75 105.5) (end 124.3 105.5) (width 0.25) (layer "F.Cu") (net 23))
 (segment (start 124.3 105.5) (end 125.25 106.45) (width 0.25) (layer "F.Cu") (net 23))
 (segment (start 125.25 100.55) (end 123.3 102.5) (width 0.25) (layer "F.Cu") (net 19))
 (segment (start 123.3 102.5) (end 122.75 102.5) (width 0.25) (layer "F.Cu") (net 19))
 (segment (start 125.25 94.45) (end 125.25 100.55) (width 0.25) (layer "F.Cu") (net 19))
 (segment (start 122.75 93.5) (end 124.3 93.5) (width 0.25) (layer "F.Cu") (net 19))
 (segment (start 124.3 93.5) (end 125.25 94.45) (width 0.25) (layer "F.Cu") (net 19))
 (segment (start 125.25 83.45) (end 125.25 88.55) (width 0.25) (layer "F.Cu") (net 15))
 (segment (start 125.25 88.55) (end 123.3 90.5) (width 0.25) (layer "F.Cu") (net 15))
 (segment (start 123.3 90.5) (end 122.75 90.5) (width 0.25) (layer "F.Cu") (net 15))
 (segment (start 122.75 81.5) (end 123.3 81.5) (width 0.25) (layer "F.Cu") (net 15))
 (segment (start 123.3 81.5) (end 125.25 83.45) (width 0.25) (layer "F.Cu") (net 15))
 (segment (start 125.25 70.45) (end 125.25 76.55) (width 0.25) (layer "F.Cu") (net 9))
 (segment (start 125.25 76.55) (end 123.3 78.5) (width 0.25) (layer "F.Cu") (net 9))
 (segment (start 123.3 78.5) (end 122.75 78.5) (width 0.25) (layer "F.Cu") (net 9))
 (segment (start 122.75 69.5) (end 124.3 69.5) (width 0.25) (layer "F.Cu") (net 9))
 (segment (start 124.3 69.5) (end 125.25 70.45) (width 0.25) (layer "F.Cu") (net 9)))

